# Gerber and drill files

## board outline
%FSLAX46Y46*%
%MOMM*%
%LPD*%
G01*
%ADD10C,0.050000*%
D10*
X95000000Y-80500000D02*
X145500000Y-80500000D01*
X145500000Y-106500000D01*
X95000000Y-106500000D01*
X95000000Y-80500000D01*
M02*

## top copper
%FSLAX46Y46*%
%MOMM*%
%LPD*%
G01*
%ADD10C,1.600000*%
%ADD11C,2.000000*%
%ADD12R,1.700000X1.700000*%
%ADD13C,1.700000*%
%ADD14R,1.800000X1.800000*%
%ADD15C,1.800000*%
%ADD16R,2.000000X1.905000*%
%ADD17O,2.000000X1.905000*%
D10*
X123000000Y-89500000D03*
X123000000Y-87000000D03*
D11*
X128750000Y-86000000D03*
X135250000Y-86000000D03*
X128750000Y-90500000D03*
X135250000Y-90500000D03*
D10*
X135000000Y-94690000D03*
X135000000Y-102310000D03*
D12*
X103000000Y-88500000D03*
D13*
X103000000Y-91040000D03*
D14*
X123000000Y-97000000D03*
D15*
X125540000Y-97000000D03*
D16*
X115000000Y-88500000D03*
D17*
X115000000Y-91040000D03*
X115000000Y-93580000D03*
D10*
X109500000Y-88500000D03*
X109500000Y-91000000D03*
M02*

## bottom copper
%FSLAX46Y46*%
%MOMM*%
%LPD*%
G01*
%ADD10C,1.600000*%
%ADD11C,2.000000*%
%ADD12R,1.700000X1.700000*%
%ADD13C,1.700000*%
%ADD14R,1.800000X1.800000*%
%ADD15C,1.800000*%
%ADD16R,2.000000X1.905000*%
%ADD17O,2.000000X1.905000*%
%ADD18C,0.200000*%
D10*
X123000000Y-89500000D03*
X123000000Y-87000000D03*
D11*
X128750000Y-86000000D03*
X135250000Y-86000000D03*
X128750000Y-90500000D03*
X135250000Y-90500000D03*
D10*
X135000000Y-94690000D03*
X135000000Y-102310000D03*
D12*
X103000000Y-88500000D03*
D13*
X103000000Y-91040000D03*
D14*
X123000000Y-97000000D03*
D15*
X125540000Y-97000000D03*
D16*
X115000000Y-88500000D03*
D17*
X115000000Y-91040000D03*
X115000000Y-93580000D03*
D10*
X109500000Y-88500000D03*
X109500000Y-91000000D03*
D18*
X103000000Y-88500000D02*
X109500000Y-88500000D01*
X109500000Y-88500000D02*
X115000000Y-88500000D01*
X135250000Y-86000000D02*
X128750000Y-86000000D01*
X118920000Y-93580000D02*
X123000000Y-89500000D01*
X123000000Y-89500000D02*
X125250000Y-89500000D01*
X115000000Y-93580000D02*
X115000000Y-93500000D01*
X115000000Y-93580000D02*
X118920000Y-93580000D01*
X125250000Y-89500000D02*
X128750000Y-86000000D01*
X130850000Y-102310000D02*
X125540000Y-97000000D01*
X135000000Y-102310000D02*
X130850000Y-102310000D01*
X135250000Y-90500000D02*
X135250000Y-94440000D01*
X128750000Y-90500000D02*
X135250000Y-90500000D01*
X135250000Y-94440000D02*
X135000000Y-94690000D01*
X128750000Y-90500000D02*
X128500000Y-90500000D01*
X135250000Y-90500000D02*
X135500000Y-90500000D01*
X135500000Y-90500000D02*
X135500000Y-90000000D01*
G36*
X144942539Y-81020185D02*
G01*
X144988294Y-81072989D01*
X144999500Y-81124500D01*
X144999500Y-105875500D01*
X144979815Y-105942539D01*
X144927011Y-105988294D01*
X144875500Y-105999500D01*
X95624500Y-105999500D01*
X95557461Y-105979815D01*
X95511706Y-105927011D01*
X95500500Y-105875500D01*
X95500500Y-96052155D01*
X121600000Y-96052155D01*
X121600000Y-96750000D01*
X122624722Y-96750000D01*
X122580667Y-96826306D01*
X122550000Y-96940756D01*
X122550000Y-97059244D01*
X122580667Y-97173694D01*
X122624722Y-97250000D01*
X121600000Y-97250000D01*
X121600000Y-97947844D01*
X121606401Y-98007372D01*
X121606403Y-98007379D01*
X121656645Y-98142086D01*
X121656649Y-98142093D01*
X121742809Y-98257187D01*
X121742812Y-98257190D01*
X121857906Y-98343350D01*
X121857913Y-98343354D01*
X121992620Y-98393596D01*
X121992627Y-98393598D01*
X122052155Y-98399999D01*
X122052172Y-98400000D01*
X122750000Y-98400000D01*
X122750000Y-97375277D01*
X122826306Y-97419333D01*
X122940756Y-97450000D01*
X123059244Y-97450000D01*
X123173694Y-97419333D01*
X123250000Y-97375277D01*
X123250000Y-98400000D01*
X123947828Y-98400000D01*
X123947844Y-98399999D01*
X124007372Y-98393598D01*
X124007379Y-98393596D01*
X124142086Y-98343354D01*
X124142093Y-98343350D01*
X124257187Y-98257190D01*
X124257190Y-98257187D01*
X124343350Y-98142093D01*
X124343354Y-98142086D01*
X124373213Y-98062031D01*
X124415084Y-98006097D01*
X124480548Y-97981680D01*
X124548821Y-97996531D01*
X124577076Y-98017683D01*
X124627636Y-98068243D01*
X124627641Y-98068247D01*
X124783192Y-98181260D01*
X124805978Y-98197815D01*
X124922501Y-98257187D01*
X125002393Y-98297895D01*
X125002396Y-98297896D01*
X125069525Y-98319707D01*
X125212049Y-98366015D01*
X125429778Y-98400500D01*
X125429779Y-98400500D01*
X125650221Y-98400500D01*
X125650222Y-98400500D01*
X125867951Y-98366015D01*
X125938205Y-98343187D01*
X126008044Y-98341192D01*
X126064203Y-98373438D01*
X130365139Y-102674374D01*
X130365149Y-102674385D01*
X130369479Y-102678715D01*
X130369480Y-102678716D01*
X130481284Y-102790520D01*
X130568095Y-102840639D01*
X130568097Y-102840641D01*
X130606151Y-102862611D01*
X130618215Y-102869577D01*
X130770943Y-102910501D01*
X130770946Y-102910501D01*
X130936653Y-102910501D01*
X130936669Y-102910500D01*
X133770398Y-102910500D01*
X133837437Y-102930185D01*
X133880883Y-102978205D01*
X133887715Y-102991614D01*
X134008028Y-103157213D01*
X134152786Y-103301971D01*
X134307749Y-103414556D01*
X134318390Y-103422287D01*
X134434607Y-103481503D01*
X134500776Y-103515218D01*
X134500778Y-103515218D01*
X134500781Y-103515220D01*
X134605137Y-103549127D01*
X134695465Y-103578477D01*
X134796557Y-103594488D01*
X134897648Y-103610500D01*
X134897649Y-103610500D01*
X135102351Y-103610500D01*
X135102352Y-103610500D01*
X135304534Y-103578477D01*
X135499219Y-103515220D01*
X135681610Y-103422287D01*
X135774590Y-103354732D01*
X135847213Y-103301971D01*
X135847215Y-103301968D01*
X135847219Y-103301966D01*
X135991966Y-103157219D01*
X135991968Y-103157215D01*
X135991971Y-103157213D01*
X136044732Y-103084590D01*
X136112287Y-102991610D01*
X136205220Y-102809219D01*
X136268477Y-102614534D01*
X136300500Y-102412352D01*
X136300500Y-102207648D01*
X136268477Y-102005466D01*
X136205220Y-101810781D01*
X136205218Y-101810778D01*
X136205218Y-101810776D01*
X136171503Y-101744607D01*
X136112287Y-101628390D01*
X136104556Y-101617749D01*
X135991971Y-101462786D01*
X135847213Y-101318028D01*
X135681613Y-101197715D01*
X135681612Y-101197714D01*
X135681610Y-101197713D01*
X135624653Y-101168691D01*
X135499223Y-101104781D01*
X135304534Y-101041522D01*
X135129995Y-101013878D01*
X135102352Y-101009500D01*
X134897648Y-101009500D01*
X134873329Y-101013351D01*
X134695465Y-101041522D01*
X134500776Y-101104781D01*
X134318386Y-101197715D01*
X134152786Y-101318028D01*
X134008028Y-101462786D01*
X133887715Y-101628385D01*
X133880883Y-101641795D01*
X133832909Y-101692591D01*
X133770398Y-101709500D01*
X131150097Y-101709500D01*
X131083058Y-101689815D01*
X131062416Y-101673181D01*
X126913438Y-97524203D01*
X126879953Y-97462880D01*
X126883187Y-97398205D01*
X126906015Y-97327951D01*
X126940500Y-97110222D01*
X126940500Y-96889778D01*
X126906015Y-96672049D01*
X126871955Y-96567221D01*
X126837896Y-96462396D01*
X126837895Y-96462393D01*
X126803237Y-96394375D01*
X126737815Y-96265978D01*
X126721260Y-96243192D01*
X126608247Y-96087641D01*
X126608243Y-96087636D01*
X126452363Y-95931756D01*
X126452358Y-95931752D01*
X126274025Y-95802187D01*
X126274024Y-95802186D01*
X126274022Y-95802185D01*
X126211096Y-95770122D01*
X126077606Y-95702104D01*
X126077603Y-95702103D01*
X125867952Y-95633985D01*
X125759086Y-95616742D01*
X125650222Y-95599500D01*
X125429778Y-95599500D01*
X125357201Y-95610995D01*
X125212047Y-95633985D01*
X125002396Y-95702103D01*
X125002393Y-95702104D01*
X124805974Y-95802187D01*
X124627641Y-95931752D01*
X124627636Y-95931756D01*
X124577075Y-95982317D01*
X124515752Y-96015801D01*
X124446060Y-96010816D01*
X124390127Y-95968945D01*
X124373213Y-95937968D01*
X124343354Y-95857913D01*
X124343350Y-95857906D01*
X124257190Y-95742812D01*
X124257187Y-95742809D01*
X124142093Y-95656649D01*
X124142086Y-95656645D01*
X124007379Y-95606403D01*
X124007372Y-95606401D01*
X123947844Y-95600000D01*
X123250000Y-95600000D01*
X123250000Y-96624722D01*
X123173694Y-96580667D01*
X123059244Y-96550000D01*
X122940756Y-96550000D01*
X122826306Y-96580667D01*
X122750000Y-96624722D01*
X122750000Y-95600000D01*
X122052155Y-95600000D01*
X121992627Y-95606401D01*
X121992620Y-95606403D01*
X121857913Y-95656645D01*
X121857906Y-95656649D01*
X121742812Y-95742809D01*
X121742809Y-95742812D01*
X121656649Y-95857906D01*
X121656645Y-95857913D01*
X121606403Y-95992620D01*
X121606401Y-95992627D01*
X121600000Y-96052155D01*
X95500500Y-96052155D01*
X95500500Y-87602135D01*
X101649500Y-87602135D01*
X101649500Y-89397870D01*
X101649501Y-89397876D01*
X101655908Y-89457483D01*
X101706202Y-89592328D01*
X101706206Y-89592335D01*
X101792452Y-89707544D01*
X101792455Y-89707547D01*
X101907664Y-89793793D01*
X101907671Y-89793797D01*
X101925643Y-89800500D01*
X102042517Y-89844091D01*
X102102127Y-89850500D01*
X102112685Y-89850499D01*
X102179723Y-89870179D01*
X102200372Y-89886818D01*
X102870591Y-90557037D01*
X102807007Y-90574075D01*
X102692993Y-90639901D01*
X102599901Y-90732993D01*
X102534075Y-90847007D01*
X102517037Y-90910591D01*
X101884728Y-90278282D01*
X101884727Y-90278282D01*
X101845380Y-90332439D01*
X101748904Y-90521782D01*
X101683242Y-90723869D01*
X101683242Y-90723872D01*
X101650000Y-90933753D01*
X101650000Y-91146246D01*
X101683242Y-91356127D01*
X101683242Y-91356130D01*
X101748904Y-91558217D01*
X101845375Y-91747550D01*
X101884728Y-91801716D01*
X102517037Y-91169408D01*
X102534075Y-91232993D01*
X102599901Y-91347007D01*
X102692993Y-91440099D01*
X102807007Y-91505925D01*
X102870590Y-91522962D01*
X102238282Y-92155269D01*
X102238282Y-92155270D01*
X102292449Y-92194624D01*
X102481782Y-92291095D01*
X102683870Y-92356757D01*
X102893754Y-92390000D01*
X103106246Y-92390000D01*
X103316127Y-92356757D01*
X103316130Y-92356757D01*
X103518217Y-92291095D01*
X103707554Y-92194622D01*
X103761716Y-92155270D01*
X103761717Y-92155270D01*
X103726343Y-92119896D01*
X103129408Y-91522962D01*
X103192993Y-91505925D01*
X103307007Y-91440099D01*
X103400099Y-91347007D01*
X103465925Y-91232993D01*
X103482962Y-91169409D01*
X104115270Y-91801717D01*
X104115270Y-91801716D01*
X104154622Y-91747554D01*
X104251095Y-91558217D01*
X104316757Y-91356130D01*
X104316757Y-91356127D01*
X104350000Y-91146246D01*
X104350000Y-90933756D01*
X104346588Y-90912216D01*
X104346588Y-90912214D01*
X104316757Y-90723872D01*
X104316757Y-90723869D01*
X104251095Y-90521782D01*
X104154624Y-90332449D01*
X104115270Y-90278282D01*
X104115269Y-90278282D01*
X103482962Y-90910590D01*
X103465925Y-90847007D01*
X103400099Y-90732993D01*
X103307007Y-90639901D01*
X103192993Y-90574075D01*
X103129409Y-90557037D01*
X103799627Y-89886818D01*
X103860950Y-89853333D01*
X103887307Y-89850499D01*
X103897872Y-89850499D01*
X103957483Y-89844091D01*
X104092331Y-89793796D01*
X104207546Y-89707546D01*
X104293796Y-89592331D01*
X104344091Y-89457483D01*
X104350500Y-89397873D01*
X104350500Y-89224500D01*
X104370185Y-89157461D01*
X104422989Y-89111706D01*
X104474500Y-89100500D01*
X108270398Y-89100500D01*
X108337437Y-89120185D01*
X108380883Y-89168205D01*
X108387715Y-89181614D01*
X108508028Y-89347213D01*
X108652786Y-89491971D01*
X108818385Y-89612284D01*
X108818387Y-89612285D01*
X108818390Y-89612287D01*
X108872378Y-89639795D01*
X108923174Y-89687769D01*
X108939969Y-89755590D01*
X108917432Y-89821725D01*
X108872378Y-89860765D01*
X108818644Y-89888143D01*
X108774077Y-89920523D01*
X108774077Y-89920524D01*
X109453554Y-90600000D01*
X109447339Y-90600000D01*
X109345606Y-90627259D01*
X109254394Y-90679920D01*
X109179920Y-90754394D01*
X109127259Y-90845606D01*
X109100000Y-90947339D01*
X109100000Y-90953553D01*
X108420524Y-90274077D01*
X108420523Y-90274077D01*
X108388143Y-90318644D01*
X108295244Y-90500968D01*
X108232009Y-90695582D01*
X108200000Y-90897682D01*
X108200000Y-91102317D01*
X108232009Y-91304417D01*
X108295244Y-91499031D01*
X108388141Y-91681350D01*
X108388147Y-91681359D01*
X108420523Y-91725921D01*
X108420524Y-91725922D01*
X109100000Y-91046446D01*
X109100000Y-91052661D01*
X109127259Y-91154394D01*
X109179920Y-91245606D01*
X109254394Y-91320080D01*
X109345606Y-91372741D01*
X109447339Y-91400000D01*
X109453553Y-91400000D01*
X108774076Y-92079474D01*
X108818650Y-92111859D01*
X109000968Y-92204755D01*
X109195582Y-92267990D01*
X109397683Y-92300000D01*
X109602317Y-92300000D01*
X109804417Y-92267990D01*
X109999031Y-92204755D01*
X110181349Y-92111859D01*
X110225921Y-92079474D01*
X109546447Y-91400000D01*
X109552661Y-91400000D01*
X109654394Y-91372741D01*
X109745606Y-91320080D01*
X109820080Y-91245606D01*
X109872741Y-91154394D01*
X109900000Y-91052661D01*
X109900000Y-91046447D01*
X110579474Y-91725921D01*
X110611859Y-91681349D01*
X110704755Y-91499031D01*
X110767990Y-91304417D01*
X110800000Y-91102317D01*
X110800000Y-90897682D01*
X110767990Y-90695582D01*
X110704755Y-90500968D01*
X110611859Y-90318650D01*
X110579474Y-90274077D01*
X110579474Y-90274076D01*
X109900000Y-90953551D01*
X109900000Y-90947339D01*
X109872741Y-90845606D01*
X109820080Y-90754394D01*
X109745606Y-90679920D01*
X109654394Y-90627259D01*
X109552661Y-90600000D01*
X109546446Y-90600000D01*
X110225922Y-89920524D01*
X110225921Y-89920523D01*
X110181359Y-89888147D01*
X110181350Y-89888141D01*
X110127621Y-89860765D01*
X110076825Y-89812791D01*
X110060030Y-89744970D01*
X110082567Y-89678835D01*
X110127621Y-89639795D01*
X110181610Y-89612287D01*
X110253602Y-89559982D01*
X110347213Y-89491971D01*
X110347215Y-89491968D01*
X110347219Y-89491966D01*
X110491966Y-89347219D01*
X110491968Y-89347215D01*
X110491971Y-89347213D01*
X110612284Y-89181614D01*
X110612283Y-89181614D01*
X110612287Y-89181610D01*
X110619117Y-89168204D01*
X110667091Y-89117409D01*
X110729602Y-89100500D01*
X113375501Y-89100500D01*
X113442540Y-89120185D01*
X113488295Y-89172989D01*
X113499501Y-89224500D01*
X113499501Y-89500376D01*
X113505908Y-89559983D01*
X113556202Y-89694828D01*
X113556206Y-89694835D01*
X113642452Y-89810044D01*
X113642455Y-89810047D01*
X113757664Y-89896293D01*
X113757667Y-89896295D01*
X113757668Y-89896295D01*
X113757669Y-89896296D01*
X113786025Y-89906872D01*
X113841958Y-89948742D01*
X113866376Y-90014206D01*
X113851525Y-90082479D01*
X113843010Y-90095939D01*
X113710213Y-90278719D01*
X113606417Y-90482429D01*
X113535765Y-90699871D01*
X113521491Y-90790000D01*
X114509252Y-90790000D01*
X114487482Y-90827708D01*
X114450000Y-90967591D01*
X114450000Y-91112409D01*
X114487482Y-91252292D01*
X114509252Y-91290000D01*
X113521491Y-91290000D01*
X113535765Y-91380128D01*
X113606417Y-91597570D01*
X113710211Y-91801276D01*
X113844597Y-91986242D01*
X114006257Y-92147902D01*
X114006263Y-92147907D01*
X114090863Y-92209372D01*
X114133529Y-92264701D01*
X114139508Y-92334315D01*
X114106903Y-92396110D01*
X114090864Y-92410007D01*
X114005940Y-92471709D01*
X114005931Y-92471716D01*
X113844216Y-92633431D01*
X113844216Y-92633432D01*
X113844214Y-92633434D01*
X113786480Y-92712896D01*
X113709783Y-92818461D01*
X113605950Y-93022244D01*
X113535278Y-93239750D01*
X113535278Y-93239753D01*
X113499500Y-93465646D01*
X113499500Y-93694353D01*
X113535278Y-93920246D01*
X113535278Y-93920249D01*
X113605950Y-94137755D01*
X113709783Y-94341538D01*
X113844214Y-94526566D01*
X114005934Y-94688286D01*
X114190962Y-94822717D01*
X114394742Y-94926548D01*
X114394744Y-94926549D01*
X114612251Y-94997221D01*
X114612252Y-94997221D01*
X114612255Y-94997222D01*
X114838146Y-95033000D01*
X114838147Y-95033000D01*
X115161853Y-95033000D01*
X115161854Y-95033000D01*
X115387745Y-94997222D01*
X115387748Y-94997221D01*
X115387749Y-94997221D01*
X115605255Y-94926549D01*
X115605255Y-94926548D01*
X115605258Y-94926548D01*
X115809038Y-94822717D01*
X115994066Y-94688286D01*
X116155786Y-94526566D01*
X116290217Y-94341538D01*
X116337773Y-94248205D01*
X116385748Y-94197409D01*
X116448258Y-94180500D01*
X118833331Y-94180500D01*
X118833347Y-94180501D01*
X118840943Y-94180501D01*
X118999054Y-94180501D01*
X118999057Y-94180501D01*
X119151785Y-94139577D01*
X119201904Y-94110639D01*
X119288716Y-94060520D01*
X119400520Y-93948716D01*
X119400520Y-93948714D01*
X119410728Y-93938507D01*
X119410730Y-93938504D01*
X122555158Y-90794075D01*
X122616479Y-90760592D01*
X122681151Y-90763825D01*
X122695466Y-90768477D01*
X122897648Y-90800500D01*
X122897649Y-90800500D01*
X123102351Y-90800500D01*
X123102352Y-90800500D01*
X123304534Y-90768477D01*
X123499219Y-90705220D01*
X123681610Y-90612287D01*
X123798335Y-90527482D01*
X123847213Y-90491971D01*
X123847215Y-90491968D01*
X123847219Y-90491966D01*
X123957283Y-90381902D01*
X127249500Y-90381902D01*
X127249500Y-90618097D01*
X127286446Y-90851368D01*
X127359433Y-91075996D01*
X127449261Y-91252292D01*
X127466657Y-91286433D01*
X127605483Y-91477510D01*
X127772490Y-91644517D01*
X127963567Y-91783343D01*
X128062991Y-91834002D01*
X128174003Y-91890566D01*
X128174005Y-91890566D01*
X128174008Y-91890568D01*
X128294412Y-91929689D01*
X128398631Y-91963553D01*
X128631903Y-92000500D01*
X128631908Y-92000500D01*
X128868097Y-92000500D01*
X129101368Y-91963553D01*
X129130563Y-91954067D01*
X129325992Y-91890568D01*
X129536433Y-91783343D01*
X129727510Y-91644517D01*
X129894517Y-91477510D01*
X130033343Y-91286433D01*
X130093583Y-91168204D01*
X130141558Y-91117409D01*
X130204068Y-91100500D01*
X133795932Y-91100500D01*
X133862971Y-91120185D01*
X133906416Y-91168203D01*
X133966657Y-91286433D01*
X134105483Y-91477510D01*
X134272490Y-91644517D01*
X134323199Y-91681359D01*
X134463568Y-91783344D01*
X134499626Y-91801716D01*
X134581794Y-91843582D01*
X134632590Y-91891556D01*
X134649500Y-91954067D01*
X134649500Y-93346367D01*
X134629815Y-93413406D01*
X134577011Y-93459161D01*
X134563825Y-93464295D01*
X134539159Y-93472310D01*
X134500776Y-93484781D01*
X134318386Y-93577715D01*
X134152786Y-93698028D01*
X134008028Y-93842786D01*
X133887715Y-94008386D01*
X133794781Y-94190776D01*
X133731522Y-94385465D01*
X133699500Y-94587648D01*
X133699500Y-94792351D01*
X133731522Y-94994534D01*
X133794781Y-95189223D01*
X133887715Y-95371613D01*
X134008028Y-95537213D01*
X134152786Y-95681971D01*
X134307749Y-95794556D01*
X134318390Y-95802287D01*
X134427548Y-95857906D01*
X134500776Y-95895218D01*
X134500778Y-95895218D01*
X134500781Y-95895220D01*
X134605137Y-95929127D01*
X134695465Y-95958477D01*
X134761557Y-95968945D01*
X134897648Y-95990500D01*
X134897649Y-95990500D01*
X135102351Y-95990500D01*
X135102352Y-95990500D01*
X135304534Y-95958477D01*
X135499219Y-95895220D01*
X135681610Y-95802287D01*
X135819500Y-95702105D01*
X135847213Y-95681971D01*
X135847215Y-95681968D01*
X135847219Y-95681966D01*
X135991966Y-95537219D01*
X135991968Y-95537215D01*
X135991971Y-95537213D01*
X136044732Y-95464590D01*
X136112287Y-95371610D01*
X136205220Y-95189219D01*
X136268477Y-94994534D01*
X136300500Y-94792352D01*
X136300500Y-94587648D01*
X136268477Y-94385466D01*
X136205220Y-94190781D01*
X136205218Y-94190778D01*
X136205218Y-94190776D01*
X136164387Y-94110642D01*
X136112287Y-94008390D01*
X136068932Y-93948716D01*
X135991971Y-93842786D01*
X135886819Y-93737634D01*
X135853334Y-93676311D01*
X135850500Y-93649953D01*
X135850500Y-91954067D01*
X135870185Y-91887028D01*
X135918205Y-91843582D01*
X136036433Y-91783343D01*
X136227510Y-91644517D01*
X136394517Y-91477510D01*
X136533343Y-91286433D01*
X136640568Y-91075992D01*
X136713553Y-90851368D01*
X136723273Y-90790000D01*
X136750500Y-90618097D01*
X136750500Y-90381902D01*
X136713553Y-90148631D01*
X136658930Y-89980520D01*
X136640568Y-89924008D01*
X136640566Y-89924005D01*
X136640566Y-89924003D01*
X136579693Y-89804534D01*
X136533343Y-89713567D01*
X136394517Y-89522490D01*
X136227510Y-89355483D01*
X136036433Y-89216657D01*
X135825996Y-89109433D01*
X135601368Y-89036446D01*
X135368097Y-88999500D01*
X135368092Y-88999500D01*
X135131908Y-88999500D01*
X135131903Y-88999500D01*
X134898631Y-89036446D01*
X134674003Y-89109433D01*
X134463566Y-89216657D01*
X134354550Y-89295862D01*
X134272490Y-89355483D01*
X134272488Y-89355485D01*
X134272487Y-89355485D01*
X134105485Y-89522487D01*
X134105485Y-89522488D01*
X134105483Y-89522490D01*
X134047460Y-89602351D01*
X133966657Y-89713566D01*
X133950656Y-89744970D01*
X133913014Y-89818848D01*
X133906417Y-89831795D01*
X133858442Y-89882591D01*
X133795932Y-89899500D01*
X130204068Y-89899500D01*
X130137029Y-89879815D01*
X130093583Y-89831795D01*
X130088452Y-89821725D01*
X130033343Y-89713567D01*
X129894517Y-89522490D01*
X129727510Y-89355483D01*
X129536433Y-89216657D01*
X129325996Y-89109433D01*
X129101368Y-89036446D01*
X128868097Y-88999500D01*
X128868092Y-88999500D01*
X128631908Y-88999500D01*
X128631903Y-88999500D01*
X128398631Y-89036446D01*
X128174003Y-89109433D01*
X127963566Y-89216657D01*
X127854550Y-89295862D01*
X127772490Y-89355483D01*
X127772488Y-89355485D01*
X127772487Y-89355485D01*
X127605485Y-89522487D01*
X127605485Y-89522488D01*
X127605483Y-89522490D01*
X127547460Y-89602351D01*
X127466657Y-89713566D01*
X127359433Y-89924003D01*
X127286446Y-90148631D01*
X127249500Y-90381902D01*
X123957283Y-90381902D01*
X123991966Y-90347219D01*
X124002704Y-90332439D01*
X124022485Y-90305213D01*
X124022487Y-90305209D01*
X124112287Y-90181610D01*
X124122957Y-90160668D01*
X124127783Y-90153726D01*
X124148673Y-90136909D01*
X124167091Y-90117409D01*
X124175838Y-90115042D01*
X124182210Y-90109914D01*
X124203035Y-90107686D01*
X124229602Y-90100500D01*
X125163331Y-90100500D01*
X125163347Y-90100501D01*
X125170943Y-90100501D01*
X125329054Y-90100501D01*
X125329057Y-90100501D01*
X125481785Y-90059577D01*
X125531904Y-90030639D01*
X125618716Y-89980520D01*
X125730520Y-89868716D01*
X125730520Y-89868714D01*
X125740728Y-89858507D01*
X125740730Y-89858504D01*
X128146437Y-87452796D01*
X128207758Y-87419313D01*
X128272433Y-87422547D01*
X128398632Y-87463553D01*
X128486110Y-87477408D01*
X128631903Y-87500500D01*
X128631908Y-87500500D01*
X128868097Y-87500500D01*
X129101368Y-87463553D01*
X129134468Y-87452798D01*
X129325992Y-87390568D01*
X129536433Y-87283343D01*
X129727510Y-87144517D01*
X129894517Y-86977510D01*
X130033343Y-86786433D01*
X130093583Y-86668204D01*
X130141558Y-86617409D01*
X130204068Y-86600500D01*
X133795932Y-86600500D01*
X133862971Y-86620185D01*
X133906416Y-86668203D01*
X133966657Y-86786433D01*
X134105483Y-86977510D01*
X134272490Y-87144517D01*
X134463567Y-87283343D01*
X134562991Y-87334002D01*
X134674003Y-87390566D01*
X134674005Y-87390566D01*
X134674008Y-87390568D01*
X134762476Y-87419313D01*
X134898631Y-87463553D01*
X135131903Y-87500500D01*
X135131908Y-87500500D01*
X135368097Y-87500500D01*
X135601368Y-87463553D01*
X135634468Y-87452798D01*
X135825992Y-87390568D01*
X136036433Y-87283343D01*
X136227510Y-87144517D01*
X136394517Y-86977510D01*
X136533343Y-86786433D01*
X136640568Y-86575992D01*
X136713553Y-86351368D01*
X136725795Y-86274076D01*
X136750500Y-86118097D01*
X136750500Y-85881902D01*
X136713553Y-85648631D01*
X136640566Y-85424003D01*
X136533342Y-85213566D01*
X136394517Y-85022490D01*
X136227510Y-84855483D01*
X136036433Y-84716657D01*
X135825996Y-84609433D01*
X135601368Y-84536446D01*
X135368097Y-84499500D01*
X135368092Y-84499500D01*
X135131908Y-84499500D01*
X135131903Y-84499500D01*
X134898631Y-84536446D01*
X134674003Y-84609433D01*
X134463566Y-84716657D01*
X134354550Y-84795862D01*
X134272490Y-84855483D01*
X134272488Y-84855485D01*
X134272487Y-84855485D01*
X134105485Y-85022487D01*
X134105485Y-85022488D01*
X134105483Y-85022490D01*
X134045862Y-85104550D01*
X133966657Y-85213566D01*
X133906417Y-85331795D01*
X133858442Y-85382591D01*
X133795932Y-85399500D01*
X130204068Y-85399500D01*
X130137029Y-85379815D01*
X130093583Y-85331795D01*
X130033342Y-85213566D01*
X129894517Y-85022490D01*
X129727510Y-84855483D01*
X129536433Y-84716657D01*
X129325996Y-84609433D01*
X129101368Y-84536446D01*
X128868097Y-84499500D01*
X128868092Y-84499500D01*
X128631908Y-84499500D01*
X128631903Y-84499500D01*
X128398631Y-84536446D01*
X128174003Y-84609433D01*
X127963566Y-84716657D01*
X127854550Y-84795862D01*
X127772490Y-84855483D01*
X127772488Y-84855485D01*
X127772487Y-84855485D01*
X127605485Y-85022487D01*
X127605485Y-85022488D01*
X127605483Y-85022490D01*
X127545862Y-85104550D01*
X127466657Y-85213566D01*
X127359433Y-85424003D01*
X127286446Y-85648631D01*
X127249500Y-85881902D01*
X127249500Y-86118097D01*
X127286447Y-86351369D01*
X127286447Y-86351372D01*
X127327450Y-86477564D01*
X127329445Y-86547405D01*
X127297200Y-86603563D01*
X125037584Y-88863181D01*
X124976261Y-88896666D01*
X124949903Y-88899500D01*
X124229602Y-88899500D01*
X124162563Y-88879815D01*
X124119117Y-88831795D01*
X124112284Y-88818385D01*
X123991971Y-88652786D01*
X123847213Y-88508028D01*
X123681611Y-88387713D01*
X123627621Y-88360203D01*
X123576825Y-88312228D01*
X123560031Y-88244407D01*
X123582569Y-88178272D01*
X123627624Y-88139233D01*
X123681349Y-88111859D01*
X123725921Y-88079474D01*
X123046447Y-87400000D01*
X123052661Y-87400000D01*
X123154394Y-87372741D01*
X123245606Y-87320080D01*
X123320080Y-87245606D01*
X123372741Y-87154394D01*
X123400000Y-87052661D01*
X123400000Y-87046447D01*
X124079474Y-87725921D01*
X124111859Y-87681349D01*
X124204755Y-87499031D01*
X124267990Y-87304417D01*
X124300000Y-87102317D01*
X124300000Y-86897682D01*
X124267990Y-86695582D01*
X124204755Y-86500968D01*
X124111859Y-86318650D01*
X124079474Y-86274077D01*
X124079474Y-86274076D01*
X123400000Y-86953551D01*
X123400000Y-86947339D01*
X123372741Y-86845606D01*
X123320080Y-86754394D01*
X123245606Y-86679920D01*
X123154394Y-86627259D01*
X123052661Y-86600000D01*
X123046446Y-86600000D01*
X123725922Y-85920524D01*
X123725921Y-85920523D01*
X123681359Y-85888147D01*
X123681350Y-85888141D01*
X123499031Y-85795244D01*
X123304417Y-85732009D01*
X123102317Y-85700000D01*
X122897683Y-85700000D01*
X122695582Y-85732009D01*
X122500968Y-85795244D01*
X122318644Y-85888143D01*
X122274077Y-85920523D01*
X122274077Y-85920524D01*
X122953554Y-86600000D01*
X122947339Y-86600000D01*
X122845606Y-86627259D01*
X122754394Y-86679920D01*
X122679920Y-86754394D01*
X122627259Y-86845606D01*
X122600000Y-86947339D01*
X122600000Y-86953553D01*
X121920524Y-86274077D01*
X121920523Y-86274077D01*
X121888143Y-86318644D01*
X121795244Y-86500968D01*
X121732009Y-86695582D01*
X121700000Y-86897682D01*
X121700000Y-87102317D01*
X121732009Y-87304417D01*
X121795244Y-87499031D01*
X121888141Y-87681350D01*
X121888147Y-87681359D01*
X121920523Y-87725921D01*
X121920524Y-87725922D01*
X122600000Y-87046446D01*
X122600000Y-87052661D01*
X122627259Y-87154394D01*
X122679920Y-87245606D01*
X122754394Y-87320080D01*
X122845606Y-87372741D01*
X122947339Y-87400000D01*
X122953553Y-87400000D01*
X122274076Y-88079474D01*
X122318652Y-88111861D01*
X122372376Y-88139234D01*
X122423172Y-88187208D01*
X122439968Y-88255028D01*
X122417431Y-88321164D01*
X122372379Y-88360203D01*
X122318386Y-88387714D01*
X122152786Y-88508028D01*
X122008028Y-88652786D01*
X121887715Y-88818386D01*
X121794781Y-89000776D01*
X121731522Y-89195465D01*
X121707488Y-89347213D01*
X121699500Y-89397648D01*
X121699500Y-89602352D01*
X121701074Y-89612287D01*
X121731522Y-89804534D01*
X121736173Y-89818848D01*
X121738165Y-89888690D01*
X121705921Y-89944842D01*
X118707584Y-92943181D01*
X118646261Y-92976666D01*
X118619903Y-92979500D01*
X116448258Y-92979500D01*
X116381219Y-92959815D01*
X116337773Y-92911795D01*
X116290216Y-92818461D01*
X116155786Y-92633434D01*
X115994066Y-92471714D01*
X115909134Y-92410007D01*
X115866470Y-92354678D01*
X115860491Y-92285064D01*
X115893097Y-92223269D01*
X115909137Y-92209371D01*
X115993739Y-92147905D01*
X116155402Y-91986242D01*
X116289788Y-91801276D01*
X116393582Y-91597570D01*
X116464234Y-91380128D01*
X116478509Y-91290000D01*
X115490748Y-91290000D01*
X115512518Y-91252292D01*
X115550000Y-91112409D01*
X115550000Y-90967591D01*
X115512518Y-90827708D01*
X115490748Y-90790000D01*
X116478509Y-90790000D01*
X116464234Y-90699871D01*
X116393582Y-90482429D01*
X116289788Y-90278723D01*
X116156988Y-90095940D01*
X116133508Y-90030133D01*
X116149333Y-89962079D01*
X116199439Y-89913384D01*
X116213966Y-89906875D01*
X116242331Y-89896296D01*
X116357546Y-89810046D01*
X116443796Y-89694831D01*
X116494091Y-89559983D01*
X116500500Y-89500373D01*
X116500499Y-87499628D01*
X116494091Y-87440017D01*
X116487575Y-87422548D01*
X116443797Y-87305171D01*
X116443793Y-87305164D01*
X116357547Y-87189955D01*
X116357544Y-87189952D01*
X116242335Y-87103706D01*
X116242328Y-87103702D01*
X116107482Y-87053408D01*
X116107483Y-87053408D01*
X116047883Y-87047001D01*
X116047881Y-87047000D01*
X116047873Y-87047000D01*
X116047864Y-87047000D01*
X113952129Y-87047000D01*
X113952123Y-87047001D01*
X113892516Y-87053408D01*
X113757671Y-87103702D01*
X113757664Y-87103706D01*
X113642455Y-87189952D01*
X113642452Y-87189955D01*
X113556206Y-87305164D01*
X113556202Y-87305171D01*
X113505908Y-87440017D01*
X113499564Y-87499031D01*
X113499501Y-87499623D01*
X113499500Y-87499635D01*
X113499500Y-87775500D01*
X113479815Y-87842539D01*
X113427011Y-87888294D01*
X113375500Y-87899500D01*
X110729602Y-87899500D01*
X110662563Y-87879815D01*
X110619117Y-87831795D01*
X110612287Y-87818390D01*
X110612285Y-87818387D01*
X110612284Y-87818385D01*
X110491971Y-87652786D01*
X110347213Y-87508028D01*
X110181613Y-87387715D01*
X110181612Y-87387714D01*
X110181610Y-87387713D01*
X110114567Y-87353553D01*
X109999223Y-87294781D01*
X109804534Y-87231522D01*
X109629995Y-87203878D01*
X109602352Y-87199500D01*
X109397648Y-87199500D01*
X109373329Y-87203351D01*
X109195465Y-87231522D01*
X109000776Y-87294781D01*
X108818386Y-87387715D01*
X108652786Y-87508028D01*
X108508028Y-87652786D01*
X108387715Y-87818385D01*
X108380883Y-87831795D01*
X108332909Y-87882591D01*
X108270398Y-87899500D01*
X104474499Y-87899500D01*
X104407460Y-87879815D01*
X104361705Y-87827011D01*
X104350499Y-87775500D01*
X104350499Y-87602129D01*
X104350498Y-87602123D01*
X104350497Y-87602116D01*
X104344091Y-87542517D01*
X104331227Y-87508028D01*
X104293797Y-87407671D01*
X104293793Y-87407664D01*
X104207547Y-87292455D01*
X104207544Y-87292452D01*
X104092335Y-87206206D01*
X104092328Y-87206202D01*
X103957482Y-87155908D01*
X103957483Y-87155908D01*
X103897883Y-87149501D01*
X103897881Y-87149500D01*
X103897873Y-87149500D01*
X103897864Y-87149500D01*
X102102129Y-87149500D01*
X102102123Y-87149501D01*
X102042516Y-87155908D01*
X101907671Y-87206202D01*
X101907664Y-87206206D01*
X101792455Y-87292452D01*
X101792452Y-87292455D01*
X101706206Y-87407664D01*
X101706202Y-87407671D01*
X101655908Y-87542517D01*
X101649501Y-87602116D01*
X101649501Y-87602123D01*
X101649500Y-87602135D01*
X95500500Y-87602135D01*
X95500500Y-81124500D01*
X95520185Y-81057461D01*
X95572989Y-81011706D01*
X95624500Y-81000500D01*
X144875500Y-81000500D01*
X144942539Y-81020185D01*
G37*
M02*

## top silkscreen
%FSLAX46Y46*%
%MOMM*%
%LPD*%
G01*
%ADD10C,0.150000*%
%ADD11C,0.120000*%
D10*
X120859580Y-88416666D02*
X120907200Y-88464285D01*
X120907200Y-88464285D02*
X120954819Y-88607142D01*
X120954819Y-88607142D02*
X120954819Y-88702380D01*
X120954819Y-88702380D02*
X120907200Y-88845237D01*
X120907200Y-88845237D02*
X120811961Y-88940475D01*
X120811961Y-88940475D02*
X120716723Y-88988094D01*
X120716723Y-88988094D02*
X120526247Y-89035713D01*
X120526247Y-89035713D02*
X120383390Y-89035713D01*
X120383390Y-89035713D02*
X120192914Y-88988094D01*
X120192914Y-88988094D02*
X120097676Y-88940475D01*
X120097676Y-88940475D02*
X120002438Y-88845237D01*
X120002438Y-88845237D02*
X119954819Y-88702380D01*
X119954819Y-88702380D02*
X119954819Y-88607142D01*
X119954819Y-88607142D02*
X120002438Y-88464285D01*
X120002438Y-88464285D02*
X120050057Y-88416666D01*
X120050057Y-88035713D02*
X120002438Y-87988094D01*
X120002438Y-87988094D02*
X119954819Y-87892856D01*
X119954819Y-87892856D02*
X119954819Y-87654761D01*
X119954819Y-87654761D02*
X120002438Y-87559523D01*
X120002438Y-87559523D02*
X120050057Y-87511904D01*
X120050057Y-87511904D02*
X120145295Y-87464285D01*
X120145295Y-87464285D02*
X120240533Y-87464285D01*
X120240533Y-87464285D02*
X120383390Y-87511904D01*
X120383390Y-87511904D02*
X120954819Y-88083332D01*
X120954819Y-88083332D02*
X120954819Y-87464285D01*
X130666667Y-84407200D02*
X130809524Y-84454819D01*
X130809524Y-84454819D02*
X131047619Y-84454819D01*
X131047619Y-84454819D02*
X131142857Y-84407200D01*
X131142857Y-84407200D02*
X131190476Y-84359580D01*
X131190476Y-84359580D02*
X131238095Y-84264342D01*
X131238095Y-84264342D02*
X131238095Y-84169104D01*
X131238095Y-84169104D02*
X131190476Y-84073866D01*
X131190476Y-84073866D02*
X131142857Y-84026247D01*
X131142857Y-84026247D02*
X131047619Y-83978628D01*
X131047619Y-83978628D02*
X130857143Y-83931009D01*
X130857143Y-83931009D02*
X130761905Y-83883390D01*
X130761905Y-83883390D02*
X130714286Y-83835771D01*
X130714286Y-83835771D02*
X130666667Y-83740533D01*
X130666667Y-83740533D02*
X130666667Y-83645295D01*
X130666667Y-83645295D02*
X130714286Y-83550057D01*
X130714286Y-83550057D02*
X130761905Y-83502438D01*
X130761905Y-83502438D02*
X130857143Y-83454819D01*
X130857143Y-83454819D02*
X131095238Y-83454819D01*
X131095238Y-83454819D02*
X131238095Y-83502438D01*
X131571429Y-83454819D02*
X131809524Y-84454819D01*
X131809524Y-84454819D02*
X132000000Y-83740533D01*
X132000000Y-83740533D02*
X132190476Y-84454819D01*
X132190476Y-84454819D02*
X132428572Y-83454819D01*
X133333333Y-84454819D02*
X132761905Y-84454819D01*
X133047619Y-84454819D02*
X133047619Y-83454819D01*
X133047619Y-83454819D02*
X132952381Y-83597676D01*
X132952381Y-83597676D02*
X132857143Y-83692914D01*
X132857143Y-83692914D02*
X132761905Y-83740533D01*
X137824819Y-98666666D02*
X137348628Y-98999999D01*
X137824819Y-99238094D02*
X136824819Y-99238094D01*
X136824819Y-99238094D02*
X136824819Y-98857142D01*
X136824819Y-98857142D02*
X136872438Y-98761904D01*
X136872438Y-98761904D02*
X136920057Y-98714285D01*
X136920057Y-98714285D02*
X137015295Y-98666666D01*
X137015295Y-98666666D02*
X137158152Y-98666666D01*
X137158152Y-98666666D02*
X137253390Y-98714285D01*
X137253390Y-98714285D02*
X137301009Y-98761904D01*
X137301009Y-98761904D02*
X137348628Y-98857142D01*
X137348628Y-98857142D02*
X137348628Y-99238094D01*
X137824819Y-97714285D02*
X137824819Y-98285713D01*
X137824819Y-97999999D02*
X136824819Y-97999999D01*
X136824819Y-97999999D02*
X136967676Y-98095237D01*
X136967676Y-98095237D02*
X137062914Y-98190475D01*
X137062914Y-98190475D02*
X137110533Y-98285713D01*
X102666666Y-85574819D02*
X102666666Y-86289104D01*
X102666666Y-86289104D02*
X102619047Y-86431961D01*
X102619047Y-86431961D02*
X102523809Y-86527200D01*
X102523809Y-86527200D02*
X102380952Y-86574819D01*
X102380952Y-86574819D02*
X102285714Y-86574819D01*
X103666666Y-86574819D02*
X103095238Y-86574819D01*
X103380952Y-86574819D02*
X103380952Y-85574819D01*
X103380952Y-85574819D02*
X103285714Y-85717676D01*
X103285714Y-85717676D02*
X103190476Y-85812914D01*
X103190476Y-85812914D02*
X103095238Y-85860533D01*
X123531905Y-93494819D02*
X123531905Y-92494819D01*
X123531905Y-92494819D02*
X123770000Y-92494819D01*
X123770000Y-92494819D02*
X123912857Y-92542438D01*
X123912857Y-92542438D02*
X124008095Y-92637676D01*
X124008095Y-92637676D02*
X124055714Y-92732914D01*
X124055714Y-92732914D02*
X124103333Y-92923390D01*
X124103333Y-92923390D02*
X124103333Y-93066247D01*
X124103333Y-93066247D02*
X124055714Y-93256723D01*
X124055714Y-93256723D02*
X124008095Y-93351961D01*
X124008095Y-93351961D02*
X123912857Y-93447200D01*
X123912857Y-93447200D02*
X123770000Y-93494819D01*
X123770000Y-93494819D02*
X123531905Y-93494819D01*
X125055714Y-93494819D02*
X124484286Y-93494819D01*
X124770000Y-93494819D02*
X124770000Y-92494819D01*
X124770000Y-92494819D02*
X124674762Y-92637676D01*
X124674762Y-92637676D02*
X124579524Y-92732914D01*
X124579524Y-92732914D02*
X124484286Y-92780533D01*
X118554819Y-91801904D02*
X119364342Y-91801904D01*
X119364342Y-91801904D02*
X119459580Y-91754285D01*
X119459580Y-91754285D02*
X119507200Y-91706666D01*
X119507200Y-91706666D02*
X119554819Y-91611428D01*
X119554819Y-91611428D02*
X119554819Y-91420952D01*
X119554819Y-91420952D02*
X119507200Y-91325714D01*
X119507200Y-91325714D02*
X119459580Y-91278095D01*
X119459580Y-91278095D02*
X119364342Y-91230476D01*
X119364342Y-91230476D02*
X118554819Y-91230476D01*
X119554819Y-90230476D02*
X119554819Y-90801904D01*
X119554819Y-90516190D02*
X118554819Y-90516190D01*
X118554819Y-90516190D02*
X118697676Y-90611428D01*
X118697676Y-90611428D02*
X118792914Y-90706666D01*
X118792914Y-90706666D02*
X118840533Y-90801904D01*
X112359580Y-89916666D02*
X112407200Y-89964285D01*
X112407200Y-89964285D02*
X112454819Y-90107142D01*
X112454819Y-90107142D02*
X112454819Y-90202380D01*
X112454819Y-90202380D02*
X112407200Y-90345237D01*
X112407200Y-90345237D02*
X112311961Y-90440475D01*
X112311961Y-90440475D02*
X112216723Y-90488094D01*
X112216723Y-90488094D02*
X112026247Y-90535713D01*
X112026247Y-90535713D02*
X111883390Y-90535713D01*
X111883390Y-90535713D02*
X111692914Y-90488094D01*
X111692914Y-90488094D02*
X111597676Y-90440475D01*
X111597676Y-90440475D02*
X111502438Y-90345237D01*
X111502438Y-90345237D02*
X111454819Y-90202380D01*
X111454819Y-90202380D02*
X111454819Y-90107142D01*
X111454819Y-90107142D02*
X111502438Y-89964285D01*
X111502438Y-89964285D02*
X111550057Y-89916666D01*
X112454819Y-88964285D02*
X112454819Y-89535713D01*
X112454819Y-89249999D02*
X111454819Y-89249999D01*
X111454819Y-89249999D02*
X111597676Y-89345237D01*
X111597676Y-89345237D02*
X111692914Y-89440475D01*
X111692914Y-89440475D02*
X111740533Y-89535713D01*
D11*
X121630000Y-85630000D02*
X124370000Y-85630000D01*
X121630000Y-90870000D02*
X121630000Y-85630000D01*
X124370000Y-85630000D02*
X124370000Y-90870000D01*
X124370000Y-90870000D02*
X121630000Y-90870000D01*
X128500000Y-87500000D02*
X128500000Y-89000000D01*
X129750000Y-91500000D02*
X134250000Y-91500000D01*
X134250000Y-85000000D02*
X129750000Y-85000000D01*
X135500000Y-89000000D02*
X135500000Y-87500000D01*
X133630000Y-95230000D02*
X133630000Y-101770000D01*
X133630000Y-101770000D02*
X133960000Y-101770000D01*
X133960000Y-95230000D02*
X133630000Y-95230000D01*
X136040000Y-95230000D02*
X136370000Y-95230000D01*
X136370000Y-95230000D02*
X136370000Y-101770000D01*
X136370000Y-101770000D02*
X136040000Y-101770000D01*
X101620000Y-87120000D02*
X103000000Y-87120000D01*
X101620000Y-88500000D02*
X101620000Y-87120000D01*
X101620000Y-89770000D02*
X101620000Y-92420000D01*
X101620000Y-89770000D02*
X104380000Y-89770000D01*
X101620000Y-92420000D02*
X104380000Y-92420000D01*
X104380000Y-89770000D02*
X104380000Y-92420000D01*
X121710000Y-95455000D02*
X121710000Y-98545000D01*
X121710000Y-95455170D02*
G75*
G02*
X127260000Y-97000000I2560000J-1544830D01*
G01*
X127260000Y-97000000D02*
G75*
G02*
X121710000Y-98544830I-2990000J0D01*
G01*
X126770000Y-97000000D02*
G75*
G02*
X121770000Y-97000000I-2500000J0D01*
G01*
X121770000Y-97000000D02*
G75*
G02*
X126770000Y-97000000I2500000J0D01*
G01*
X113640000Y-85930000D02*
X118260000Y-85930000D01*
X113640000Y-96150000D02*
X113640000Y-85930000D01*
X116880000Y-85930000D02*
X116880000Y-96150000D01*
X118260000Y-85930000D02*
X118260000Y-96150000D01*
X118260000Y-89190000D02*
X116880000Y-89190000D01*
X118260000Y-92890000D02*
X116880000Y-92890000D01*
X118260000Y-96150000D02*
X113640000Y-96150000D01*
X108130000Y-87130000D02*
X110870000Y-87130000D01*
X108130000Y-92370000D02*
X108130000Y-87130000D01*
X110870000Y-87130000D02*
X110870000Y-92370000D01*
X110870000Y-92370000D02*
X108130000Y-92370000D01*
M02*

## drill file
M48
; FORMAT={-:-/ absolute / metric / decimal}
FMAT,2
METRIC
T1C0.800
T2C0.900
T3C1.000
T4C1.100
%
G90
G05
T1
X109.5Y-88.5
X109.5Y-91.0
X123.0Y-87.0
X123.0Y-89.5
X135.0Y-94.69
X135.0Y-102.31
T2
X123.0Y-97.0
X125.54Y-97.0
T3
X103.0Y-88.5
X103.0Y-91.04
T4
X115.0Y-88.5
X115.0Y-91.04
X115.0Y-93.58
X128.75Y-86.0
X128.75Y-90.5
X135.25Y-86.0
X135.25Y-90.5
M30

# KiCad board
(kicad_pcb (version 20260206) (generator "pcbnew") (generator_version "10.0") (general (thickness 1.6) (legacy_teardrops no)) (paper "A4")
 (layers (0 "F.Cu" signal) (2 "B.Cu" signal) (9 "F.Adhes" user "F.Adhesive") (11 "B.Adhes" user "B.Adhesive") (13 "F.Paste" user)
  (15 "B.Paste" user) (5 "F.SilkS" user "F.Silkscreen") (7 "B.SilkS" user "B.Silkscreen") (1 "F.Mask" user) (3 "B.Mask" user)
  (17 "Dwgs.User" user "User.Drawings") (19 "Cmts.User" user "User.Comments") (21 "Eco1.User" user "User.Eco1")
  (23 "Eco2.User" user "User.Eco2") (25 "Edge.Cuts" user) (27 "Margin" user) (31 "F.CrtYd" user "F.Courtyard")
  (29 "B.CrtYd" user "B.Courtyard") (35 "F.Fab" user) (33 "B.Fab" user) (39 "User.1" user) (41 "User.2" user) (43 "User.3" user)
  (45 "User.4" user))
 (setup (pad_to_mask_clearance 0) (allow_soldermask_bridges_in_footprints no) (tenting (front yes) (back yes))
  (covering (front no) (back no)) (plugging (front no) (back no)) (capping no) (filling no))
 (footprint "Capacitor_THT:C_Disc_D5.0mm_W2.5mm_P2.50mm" (layer "F.Cu") (at 123 89.5 90)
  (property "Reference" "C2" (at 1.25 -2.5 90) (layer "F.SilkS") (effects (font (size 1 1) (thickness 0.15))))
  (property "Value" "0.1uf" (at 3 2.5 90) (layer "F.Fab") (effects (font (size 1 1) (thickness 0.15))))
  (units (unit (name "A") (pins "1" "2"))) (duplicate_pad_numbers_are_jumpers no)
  (fp_line (start 3.87 -1.37) (end 3.87 1.37) (stroke (width 0.12) (type solid)) (layer "F.SilkS"))
  (fp_line (start -1.37 -1.37) (end 3.87 -1.37) (stroke (width 0.12) (type solid)) (layer "F.SilkS"))
  (fp_line (start 3.87 1.37) (end -1.37 1.37) (stroke (width 0.12) (type solid)) (layer "F.SilkS"))
  (fp_line (start -1.37 1.37) (end -1.37 -1.37) (stroke (width 0.12) (type solid)) (layer "F.SilkS"))
  (pad "1" thru_hole circle (at 0 0 90) (size 1.6 1.6) (drill 0.8) (layers "*.Cu" "*.Mask") (remove_unused_layers no) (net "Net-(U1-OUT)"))
  (pad "2" thru_hole circle (at 2.5 0 90) (size 1.6 1.6) (drill 0.8) (layers "*.Cu" "*.Mask") (remove_unused_layers no) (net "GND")))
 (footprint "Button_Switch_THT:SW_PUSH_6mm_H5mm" (layer "F.Cu") (at 128.75 86)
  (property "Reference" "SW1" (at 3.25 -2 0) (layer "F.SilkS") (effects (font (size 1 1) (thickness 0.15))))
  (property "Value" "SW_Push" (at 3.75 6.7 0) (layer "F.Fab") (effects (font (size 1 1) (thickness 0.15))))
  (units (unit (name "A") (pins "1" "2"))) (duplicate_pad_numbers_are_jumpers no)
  (fp_line (start -0.25 1.5) (end -0.25 3) (stroke (width 0.12) (type solid)) (layer "F.SilkS"))
  (fp_line (start 1 5.5) (end 5.5 5.5) (stroke (width 0.12) (type solid)) (layer "F.SilkS"))
  (fp_line (start 5.5 -1) (end 1 -1) (stroke (width 0.12) (type solid)) (layer "F.SilkS"))
  (fp_line (start 6.75 3) (end 6.75 1.5) (stroke (width 0.12) (type solid)) (layer "F.SilkS"))
  (pad "1" thru_hole circle (at 0 0 90) (size 2 2) (drill 1.1) (layers "*.Cu" "*.Mask") (remove_unused_layers no) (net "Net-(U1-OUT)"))
  (pad "1" thru_hole circle (at 6.5 0 90) (size 2 2) (drill 1.1) (layers "*.Cu" "*.Mask") (remove_unused_layers no) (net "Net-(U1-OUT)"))
  (pad "2" thru_hole circle (at 0 4.5 90) (size 2 2) (drill 1.1) (layers "*.Cu" "*.Mask") (remove_unused_layers no) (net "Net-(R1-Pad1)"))
  (pad "2" thru_hole circle (at 6.5 4.5 90) (size 2 2) (drill 1.1) (layers "*.Cu" "*.Mask") (remove_unused_layers no) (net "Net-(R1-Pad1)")))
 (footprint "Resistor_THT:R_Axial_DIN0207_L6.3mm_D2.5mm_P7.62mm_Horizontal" (layer "F.Cu") (at 135 94.69 -90)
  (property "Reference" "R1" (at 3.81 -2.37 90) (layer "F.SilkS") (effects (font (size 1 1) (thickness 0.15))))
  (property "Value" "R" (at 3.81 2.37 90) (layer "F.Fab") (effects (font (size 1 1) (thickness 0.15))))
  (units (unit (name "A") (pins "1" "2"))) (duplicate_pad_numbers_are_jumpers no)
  (fp_line (start 0.54 1.37) (end 7.08 1.37) (stroke (width 0.12) (type solid)) (layer "F.SilkS"))
  (fp_line (start 7.08 1.37) (end 7.08 1.04) (stroke (width 0.12) (type solid)) (layer "F.SilkS"))
  (fp_line (start 0.54 1.04) (end 0.54 1.37) (stroke (width 0.12) (type solid)) (layer "F.SilkS"))
  (fp_line (start 0.54 -1.04) (end 0.54 -1.37) (stroke (width 0.12) (type solid)) (layer "F.SilkS"))
  (fp_line (start 0.54 -1.37) (end 7.08 -1.37) (stroke (width 0.12) (type solid)) (layer "F.SilkS"))
  (fp_line (start 7.08 -1.37) (end 7.08 -1.04) (stroke (width 0.12) (type solid)) (layer "F.SilkS"))
  (pad "1" thru_hole circle (at 0 0 270) (size 1.6 1.6) (drill 0.8) (layers "*.Cu" "*.Mask") (remove_unused_layers no) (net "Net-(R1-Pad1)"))
  (pad "2" thru_hole circle (at 7.62 0 270) (size 1.6 1.6) (drill 0.8) (layers "*.Cu" "*.Mask") (remove_unused_layers no) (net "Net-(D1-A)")))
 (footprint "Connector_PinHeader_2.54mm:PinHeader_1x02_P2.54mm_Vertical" (layer "F.Cu") (at 103 88.5)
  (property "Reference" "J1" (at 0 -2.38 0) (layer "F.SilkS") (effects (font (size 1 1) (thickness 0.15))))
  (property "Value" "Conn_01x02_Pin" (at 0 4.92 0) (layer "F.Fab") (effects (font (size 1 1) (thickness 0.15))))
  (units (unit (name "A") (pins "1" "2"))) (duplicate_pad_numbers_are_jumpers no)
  (fp_line (start -1.38 -1.38) (end 0 -1.38) (stroke (width 0.12) (type solid)) (layer "F.SilkS"))
  (fp_line (start -1.38 0) (end -1.38 -1.38) (stroke (width 0.12) (type solid)) (layer "F.SilkS"))
  (fp_line (start -1.38 1.27) (end -1.38 3.92) (stroke (width 0.12) (type solid)) (layer "F.SilkS"))
  (fp_line (start -1.38 1.27) (end 1.38 1.27) (stroke (width 0.12) (type solid)) (layer "F.SilkS"))
  (fp_line (start -1.38 3.92) (end 1.38 3.92) (stroke (width 0.12) (type solid)) (layer "F.SilkS"))
  (fp_line (start 1.38 1.27) (end 1.38 3.92) (stroke (width 0.12) (type solid)) (layer "F.SilkS"))
  (pad "1" thru_hole rect (at 0 0) (size 1.7 1.7) (drill 1) (layers "*.Cu" "*.Mask") (remove_unused_layers no) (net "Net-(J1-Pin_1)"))
  (pad "2" thru_hole circle (at 0 2.54) (size 1.7 1.7) (drill 1) (layers "*.Cu" "*.Mask") (remove_unused_layers no) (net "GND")))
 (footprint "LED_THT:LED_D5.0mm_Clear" (layer "F.Cu") (at 123 97)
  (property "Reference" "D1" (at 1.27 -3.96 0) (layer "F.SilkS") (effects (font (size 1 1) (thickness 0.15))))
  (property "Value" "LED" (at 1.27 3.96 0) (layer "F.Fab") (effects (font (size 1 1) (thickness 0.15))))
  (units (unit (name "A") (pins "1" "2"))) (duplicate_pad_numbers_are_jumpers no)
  (fp_line (start -1.29 -1.545) (end -1.29 1.545) (stroke (width 0.12) (type solid)) (layer "F.SilkS"))
  (fp_arc (start -1.29 -1.54483) (mid 2.071779 -2.880495) (end 4.26 0) (stroke (width 0.12) (type solid)) (layer "F.SilkS"))
  (fp_arc (start 4.26 0) (mid 2.071779 2.880495) (end -1.29 1.54483) (stroke (width 0.12) (type solid)) (layer "F.SilkS"))
  (fp_circle (center 1.27 0) (end 3.77 0) (stroke (width 0.12) (type solid)) (fill no) (layer "F.SilkS"))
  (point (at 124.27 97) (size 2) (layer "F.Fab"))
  (pad "1" thru_hole rect (at 0 0) (size 1.8 1.8) (drill 0.9) (layers "*.Cu" "*.Mask") (remove_unused_layers no) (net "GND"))
  (pad "2" thru_hole circle (at 2.54 0) (size 1.8 1.8) (drill 0.9) (layers "*.Cu" "*.Mask") (remove_unused_layers no) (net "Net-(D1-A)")))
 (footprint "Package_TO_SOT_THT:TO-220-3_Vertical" (layer "F.Cu") (at 115 88.5 -90)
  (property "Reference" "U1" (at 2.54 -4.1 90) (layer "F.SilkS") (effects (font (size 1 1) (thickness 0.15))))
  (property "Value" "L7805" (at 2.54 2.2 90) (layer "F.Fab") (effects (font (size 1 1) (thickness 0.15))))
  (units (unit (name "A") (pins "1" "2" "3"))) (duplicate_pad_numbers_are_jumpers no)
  (fp_line (start -2.57 1.36) (end -2.57 -3.26) (stroke (width 0.12) (type solid)) (layer "F.SilkS"))
  (fp_line (start 7.65 1.36) (end -2.57 1.36) (stroke (width 0.12) (type solid)) (layer "F.SilkS"))
  (fp_line (start -2.57 -1.88) (end 7.65 -1.88) (stroke (width 0.12) (type solid)) (layer "F.SilkS"))
  (fp_line (start -2.57 -3.26) (end 7.65 -3.26) (stroke (width 0.12) (type solid)) (layer "F.SilkS"))
  (fp_line (start 0.69 -3.26) (end 0.69 -1.88) (stroke (width 0.12) (type solid)) (layer "F.SilkS"))
  (fp_line (start 4.39 -3.26) (end 4.39 -1.88) (stroke (width 0.12) (type solid)) (layer "F.SilkS"))
  (fp_line (start 7.65 -3.26) (end 7.65 1.36) (stroke (width 0.12) (type solid)) (layer "F.SilkS"))
  (pad "1" thru_hole rect (at 0 0 270) (size 1.905 2) (drill 1.1) (layers "*.Cu" "*.Mask") (remove_unused_layers no) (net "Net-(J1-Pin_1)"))
  (pad "2" thru_hole oval (at 2.54 0 270) (size 1.905 2) (drill 1.1) (layers "*.Cu" "*.Mask") (remove_unused_layers no) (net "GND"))
  (pad "3" thru_hole oval (at 5.08 0 270) (size 1.905 2) (drill 1.1) (layers "*.Cu" "*.Mask") (remove_unused_layers no) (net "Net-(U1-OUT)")))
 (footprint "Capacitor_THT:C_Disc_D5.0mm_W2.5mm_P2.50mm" (layer "F.Cu") (at 109.5 88.5 -90)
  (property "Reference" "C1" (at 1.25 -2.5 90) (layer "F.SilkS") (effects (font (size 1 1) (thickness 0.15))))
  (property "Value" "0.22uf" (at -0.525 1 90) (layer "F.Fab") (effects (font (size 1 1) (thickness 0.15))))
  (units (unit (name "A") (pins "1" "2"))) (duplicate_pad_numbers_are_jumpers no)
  (fp_line (start -1.37 1.37) (end -1.37 -1.37) (stroke (width 0.12) (type solid)) (layer "F.SilkS"))
  (fp_line (start 3.87 1.37) (end -1.37 1.37) (stroke (width 0.12) (type solid)) (layer "F.SilkS"))
  (fp_line (start -1.37 -1.37) (end 3.87 -1.37) (stroke (width 0.12) (type solid)) (layer "F.SilkS"))
  (fp_line (start 3.87 -1.37) (end 3.87 1.37) (stroke (width 0.12) (type solid)) (layer "F.SilkS"))
  (pad "1" thru_hole circle (at 0 0 270) (size 1.6 1.6) (drill 0.8) (layers "*.Cu" "*.Mask") (remove_unused_layers no)
   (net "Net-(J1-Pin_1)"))
  (pad "2" thru_hole circle (at 2.5 0 270) (size 1.6 1.6) (drill 0.8) (layers "*.Cu" "*.Mask") (remove_unused_layers no) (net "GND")))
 (gr_rect (start 95 80.5) (end 145.5 106.5) (stroke (width 0.05) (type default)) (fill no) (layer "Edge.Cuts"))
 (segment (start 103 88.5) (end 109.5 88.5) (width 0.2) (layer "B.Cu") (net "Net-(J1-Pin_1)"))
 (segment (start 109.5 88.5) (end 115 88.5) (width 0.2) (layer "B.Cu") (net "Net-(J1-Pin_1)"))
 (segment (start 135.25 86) (end 128.75 86) (width 0.2) (layer "B.Cu") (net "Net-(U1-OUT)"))
 (segment (start 118.92 93.58) (end 123 89.5) (width 0.2) (layer "B.Cu") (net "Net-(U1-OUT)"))
 (segment (start 123 89.5) (end 125.25 89.5) (width 0.2) (layer "B.Cu") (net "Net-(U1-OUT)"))
 (segment (start 115 93.58) (end 115 93.5) (width 0.2) (layer "B.Cu") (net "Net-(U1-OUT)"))
 (segment (start 115 93.58) (end 118.92 93.58) (width 0.2) (layer "B.Cu") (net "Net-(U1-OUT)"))
 (segment (start 125.25 89.5) (end 128.75 86) (width 0.2) (layer "B.Cu") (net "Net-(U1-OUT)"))
 (segment (start 130.85 102.31) (end 125.54 97) (width 0.2) (layer "B.Cu") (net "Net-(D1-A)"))
 (segment (start 135 102.31) (end 130.85 102.31) (width 0.2) (layer "B.Cu") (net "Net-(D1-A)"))
 (segment (start 135.25 90.5) (end 135.25 94.44) (width 0.2) (layer "B.Cu") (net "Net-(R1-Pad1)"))
 (segment (start 128.75 90.5) (end 135.25 90.5) (width 0.2) (layer "B.Cu") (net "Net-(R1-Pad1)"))
 (segment (start 135.25 94.44) (end 135 94.69) (width 0.2) (layer "B.Cu") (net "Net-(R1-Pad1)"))
 (segment (start 128.75 90.5) (end 128.5 90.5) (width 0.2) (layer "B.Cu") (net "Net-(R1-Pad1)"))
 (segment (start 135.25 90.5) (end 135.5 90.5) (width 0.2) (layer "B.Cu") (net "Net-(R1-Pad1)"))
 (segment (start 135.5 90.5) (end 135.5 90) (width 0.2) (layer "B.Cu") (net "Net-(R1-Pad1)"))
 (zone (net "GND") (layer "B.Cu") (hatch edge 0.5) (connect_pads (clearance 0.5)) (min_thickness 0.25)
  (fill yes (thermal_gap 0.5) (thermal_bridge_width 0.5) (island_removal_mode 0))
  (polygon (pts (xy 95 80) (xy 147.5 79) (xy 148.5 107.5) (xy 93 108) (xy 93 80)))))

